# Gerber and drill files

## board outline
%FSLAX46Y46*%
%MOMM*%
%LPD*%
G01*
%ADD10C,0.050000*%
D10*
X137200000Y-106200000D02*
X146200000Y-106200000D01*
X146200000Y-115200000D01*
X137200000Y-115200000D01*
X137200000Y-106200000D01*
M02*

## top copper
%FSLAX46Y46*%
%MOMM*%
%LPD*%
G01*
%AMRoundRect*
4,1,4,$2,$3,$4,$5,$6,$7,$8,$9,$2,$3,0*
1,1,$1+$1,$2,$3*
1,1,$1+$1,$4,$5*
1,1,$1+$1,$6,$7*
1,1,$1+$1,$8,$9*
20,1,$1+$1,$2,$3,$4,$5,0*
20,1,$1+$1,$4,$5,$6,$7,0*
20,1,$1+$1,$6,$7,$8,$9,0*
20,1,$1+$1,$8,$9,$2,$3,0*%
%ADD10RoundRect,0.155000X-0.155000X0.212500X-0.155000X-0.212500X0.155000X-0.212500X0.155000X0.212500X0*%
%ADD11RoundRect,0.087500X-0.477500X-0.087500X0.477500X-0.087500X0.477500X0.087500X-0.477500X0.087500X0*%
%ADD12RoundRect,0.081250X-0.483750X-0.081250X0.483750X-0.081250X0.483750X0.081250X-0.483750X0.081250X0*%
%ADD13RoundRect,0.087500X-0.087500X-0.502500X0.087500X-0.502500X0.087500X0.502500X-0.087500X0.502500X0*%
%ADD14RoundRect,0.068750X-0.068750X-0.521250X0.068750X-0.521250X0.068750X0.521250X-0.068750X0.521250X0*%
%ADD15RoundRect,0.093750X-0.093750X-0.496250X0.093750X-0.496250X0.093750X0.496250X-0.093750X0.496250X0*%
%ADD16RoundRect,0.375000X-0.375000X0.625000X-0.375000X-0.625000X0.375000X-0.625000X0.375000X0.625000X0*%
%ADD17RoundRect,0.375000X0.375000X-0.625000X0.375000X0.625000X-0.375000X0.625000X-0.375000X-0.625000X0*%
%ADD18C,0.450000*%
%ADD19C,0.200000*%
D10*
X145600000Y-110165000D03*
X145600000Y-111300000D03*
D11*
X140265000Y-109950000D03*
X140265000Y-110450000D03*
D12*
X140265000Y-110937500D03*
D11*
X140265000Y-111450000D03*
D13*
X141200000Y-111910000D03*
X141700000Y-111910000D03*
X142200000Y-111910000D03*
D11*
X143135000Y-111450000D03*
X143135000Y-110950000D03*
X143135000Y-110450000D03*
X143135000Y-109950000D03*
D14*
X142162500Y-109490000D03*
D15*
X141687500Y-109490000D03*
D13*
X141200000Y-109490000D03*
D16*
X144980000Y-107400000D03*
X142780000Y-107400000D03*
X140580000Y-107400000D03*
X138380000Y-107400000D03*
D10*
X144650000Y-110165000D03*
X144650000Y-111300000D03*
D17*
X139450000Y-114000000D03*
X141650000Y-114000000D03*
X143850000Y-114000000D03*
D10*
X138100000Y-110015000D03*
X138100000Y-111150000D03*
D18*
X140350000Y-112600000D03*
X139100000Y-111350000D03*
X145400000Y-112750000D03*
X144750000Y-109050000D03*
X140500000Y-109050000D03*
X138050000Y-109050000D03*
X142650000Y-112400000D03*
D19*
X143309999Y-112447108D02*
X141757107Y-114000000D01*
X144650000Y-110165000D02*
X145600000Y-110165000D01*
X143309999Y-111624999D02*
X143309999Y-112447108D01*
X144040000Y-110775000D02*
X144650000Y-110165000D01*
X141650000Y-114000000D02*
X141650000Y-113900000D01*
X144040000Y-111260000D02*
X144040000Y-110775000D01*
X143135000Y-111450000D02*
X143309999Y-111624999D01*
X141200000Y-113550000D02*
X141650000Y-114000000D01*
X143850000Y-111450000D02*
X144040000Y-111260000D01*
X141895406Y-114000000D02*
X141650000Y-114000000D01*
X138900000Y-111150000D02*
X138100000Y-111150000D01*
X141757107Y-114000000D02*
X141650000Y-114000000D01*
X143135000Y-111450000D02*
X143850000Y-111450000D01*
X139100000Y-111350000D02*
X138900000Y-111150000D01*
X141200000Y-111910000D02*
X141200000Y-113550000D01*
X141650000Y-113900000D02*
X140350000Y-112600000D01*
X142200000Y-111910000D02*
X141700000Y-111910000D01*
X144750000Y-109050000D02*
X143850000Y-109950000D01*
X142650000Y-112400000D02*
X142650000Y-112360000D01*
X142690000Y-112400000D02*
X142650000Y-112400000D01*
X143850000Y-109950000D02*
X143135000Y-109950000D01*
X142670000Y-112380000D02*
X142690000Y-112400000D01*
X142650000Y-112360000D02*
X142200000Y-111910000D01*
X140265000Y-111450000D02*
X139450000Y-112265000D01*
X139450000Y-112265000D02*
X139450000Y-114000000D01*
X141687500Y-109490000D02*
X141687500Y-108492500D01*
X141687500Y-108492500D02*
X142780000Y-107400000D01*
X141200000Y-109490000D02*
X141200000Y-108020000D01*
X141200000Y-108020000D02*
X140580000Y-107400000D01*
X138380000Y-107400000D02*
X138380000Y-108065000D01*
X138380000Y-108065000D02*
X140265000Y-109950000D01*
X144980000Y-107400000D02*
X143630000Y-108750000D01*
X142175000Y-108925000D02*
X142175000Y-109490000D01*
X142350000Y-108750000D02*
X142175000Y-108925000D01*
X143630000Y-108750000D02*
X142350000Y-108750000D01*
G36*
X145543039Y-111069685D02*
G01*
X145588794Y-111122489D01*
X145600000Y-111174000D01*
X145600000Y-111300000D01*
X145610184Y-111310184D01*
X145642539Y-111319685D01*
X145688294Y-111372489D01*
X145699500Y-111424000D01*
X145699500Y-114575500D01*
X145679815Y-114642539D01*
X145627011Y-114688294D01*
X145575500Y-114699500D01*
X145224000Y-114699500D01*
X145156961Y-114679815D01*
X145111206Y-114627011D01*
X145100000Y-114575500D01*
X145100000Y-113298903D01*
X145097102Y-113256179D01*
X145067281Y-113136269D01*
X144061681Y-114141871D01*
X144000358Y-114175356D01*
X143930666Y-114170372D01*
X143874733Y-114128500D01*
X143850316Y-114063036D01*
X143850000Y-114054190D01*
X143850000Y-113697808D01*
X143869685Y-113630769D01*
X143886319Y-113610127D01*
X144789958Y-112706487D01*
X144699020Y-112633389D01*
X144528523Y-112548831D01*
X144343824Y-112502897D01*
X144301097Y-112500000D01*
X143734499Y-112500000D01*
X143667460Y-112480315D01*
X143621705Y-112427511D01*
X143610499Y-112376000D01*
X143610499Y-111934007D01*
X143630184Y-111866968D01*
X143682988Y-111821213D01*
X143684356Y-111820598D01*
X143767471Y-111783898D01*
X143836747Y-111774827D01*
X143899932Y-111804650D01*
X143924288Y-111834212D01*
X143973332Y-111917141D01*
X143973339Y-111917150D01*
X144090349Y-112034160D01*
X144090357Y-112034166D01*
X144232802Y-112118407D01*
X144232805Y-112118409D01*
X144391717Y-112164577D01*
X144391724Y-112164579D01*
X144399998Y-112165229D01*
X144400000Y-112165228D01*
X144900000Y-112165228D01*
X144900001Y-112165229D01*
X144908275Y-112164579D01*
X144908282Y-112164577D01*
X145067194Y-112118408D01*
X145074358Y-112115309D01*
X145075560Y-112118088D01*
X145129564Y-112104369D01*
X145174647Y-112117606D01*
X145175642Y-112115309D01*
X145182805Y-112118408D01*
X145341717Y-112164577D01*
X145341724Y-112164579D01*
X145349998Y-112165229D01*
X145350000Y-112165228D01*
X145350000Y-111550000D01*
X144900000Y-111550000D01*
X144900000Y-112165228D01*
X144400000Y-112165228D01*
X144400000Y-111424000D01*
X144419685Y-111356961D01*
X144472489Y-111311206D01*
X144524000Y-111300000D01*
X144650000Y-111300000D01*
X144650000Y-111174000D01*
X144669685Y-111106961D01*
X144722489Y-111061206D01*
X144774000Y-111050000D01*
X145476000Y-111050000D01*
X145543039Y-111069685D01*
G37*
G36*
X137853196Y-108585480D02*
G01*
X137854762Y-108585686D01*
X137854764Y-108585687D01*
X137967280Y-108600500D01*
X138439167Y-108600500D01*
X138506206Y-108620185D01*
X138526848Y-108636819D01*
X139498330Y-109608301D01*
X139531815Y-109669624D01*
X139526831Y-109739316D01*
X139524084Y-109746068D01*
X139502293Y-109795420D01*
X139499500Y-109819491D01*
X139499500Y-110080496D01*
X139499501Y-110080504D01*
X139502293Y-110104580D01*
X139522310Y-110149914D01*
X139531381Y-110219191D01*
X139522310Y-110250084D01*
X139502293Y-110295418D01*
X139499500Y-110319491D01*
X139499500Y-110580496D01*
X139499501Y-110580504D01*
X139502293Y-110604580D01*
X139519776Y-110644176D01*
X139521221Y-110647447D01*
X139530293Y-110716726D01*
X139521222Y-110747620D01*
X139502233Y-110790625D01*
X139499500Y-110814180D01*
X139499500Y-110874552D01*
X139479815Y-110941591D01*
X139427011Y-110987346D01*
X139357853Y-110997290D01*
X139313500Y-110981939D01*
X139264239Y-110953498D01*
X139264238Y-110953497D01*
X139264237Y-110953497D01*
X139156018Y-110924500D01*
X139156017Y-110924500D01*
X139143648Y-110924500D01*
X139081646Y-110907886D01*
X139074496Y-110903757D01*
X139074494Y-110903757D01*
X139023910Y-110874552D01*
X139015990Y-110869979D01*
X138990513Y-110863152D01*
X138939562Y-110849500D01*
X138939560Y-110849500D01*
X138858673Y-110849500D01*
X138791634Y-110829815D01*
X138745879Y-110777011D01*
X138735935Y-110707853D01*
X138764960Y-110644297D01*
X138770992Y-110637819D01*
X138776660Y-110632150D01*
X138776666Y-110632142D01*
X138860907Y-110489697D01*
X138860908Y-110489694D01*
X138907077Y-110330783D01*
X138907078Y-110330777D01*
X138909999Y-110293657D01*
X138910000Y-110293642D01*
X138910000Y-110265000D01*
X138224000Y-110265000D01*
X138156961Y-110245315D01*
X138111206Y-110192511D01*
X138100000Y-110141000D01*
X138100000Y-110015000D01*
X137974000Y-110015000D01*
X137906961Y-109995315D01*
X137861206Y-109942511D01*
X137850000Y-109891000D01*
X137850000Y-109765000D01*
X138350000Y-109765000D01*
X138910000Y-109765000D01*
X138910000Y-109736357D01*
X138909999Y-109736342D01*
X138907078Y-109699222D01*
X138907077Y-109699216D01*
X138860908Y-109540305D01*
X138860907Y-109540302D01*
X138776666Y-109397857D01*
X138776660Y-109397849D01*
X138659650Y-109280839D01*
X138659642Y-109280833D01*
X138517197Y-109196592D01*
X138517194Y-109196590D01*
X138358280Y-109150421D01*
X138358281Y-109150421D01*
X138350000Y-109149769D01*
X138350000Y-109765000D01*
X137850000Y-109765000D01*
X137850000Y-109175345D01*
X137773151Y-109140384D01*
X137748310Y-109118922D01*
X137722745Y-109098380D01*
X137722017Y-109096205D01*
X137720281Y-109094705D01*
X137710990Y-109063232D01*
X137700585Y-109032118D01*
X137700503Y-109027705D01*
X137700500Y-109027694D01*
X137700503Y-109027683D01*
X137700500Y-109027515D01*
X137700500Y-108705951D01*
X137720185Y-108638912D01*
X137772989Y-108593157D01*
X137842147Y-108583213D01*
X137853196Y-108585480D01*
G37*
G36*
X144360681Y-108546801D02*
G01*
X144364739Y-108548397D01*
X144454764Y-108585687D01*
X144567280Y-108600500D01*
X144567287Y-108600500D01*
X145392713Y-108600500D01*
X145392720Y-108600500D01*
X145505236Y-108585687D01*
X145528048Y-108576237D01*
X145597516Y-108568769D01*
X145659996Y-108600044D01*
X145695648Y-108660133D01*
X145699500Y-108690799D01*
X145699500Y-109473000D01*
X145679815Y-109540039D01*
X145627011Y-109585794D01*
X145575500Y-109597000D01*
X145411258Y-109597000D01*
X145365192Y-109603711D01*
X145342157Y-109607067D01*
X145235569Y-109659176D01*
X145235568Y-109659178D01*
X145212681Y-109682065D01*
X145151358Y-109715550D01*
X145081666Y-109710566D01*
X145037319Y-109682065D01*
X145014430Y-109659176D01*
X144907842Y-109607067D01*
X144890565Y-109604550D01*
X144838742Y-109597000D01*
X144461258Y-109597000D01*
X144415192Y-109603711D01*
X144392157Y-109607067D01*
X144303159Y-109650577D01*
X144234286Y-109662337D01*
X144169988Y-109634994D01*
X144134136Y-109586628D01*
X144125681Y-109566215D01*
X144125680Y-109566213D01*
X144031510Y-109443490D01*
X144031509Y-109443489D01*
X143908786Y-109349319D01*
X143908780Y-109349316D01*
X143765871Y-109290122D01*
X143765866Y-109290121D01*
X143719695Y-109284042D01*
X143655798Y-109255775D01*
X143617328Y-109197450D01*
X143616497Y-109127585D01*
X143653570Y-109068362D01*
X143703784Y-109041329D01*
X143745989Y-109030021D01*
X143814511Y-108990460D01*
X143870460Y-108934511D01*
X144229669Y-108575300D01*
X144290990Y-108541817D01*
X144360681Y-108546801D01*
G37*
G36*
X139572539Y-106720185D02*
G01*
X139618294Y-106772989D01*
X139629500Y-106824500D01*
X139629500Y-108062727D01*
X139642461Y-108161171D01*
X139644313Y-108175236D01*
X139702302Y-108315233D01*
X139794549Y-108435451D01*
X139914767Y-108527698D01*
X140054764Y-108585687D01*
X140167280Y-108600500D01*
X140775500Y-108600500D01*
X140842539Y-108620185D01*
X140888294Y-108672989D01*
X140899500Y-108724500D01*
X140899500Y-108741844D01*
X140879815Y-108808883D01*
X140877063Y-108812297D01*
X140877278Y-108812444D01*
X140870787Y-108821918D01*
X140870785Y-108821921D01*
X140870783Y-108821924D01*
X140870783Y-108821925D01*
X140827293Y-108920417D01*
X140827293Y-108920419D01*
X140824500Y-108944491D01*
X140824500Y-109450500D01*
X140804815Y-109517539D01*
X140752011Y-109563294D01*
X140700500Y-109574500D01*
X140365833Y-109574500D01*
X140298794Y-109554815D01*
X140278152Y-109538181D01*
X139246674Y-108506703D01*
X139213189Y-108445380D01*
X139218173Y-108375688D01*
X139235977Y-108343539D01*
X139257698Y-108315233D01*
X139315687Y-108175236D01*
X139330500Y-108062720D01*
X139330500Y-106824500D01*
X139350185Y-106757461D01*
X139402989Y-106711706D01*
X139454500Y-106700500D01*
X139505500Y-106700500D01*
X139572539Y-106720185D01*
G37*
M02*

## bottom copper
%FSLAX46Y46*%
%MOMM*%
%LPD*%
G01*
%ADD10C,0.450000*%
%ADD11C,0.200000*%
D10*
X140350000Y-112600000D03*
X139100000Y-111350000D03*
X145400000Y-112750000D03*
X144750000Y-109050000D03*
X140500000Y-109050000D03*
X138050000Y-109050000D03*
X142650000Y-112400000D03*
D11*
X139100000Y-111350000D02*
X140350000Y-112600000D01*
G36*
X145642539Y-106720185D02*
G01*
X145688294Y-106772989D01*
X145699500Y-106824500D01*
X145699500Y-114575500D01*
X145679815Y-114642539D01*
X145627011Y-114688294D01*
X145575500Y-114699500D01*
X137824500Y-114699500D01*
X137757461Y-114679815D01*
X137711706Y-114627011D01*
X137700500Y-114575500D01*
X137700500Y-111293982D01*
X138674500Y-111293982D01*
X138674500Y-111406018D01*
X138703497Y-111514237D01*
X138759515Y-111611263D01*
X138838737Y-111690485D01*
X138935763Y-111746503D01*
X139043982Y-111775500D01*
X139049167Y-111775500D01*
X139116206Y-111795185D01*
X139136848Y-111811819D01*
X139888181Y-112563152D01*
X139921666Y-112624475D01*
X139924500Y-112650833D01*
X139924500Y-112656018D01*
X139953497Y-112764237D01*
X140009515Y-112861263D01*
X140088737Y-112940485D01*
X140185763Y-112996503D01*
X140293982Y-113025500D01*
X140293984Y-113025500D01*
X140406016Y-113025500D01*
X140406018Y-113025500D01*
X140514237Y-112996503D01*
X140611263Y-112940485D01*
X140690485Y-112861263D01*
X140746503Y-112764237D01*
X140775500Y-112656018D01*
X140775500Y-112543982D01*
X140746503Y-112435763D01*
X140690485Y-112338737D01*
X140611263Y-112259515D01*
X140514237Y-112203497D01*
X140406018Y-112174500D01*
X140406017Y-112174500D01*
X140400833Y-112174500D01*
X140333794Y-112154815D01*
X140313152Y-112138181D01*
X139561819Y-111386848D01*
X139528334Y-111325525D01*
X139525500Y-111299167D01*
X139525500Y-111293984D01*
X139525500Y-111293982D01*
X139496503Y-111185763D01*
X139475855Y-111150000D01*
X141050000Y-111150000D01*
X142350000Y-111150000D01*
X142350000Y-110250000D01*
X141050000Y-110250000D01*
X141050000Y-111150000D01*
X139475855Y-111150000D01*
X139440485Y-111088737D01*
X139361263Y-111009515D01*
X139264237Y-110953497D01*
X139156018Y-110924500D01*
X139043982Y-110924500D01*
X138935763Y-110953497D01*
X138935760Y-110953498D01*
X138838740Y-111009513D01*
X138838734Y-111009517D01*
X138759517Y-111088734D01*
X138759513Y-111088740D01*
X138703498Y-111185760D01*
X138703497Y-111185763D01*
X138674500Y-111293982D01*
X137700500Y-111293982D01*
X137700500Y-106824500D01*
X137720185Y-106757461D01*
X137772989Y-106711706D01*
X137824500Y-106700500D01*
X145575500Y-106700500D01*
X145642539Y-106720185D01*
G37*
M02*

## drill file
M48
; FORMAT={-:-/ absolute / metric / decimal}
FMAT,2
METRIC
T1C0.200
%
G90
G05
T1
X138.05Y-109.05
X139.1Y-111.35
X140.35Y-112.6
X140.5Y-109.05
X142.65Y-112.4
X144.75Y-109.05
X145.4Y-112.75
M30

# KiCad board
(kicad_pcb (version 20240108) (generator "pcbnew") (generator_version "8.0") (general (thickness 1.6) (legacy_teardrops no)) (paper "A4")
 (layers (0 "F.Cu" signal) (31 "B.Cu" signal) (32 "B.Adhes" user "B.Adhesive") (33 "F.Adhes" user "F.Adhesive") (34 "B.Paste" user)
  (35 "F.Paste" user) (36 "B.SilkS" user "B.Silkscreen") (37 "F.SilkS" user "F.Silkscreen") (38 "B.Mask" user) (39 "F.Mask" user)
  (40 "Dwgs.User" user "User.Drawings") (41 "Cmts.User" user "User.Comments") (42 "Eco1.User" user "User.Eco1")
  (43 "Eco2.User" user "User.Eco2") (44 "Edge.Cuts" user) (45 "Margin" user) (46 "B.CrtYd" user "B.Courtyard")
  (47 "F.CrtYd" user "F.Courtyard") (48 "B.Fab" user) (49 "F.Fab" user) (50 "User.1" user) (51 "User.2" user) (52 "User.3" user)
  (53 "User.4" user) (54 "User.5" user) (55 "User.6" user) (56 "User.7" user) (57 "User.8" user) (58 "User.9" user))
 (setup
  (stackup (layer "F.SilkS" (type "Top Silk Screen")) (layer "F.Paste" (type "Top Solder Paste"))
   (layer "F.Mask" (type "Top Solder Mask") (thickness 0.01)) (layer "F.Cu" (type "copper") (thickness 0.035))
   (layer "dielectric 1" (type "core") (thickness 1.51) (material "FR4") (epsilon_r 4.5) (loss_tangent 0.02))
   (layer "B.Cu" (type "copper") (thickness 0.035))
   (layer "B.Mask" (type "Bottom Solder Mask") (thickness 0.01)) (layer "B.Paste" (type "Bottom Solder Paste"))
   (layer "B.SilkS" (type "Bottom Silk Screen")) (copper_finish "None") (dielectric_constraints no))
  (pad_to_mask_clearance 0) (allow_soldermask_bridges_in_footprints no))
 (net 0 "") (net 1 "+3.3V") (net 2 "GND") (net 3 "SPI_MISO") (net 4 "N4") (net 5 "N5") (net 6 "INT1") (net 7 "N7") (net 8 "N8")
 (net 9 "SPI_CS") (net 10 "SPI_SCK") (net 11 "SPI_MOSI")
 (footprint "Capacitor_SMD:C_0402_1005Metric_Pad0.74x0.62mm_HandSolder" (layer "F.Cu") (at 145.6 110.7325 -90)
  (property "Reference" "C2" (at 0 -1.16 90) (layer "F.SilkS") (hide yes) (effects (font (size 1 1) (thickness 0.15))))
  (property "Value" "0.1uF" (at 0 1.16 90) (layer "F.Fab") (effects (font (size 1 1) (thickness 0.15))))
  (pad "1" smd roundrect (at -0.5675 0 270) (size 0.735 0.62) (layers "F.Cu" "F.Paste" "F.Mask") (roundrect_rratio 0.25) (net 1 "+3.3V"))
  (pad "2" smd roundrect (at 0.5675 0 270) (size 0.735 0.62) (layers "F.Cu" "F.Paste" "F.Mask") (roundrect_rratio 0.25) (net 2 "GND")))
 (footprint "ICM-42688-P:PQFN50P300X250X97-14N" (layer "F.Cu") (at 141.7 110.7)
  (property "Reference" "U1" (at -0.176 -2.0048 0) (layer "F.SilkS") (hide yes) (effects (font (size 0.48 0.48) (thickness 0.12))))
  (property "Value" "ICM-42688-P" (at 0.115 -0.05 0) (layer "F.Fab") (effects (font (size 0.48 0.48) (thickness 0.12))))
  (pad "1" smd roundrect (at -1.435 -0.75) (size 1.13 0.35) (layers "F.Cu" "F.Paste") (roundrect_rratio 0.25) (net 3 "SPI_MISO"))
  (pad "2" smd roundrect (at -1.435 -0.25) (size 1.13 0.35) (layers "F.Cu" "F.Paste") (roundrect_rratio 0.25) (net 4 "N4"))
  (pad "3" smd roundrect (at -1.435 0.2375) (size 1.13 0.325) (layers "F.Cu" "F.Paste") (roundrect_rratio 0.25) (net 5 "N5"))
  (pad "4" smd roundrect (at -1.435 0.75) (size 1.13 0.35) (layers "F.Cu" "F.Paste") (roundrect_rratio 0.25) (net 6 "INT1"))
  (pad "5" smd roundrect (at -0.5 1.21) (size 0.35 1.18) (layers "F.Cu" "F.Paste") (roundrect_rratio 0.25) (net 1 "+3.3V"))
  (pad "6" smd roundrect (at 0 1.21) (size 0.35 1.18) (layers "F.Cu" "F.Paste") (roundrect_rratio 0.25) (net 2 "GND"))
  (pad "7" smd roundrect (at 0.5 1.21) (size 0.35 1.18) (layers "F.Cu" "F.Paste") (roundrect_rratio 0.25) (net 2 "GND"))
  (pad "8" smd roundrect (at 1.435 0.75) (size 1.13 0.35) (layers "F.Cu" "F.Paste") (roundrect_rratio 0.25) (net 1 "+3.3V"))
  (pad "9" smd roundrect (at 1.435 0.25) (size 1.13 0.35) (layers "F.Cu" "F.Paste") (roundrect_rratio 0.25) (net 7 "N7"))
  (pad "10" smd roundrect (at 1.435 -0.25) (size 1.13 0.35) (layers "F.Cu" "F.Paste") (roundrect_rratio 0.25) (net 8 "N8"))
  (pad "11" smd roundrect (at 1.435 -0.75) (size 1.13 0.35) (layers "F.Cu" "F.Paste") (roundrect_rratio 0.25) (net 2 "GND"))
  (pad "12" smd roundrect (at 0.4625 -1.21) (size 0.275 1.18) (layers "F.Cu" "F.Paste") (roundrect_rratio 0.25) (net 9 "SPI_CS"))
  (pad "13" smd roundrect (at -0.0125 -1.21) (size 0.375 1.18) (layers "F.Cu" "F.Paste") (roundrect_rratio 0.25) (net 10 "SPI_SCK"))
  (pad "14" smd roundrect (at -0.5 -1.21) (size 0.35 1.18) (layers "F.Cu" "F.Paste") (roundrect_rratio 0.25) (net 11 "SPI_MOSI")))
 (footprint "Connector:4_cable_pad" (layer "F.Cu") (at 145.78 106.2 180)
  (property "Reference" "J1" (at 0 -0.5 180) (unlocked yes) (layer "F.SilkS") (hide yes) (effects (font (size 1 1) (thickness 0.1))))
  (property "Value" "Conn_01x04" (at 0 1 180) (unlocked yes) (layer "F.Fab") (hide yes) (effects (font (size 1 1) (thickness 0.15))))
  (pad "1" smd roundrect (at 0.8 -1.2 270) (size 2 1.5) (layers "F.Cu" "F.Paste" "F.Mask") (roundrect_rratio 0.25) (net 9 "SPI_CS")
   (thermal_bridge_angle 45))
  (pad "2" smd roundrect (at 3 -1.2 270) (size 2 1.5) (layers "F.Cu" "F.Paste" "F.Mask") (roundrect_rratio 0.25) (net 10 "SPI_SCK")
   (thermal_bridge_angle 45))
  (pad "3" smd roundrect (at 5.2 -1.2 270) (size 2 1.5) (layers "F.Cu" "F.Paste" "F.Mask") (roundrect_rratio 0.25) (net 11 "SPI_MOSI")
   (thermal_bridge_angle 45))
  (pad "4" smd roundrect (at 7.4 -1.2 270) (size 2 1.5) (layers "F.Cu" "F.Paste" "F.Mask") (roundrect_rratio 0.25) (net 3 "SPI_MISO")
   (thermal_bridge_angle 45)))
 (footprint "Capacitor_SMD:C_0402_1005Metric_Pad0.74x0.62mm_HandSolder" (layer "F.Cu") (at 144.65 110.7325 -90)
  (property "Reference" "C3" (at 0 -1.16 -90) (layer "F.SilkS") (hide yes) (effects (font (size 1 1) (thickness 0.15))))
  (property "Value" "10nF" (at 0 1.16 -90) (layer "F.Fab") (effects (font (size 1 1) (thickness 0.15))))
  (pad "1" smd roundrect (at -0.5675 0 270) (size 0.735 0.62) (layers "F.Cu" "F.Paste" "F.Mask") (roundrect_rratio 0.25) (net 1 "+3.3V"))
  (pad "2" smd roundrect (at 0.5675 0 270) (size 0.735 0.62) (layers "F.Cu" "F.Paste" "F.Mask") (roundrect_rratio 0.25) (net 2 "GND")))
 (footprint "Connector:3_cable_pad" (layer "F.Cu") (at 138.65 115.2)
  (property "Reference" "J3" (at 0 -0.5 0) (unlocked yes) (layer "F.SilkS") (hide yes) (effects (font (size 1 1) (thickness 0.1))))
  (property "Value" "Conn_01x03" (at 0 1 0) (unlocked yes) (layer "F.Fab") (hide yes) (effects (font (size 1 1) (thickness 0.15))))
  (pad "1" smd roundrect (at 0.8 -1.2 90) (size 2 1.5) (layers "F.Cu" "F.Paste" "F.Mask") (roundrect_rratio 0.25) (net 6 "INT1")
   (thermal_bridge_angle 45))
  (pad "2" smd roundrect (at 3 -1.2 90) (size 2 1.5) (layers "F.Cu" "F.Paste" "F.Mask") (roundrect_rratio 0.25) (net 1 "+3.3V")
   (thermal_bridge_angle 45))
  (pad "3" smd roundrect (at 5.2 -1.2 90) (size 2 1.5) (layers "F.Cu" "F.Paste" "F.Mask") (roundrect_rratio 0.25) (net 2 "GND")
   (thermal_bridge_angle 45)))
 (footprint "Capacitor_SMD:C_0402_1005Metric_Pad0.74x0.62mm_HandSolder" (layer "F.Cu") (at 138.1 110.5825 -90)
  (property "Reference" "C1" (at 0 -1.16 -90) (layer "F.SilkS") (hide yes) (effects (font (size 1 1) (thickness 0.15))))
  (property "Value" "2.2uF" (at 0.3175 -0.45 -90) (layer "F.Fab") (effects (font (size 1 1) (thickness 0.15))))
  (pad "1" smd roundrect (at -0.5675 0 270) (size 0.735 0.62) (layers "F.Cu" "F.Paste" "F.Mask") (roundrect_rratio 0.25) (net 2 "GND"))
  (pad "2" smd roundrect (at 0.5675 0 270) (size 0.735 0.62) (layers "F.Cu" "F.Paste" "F.Mask") (roundrect_rratio 0.25) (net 1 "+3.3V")))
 (gr_rect (start 137.2 106.2) (end 146.2 115.2) (stroke (width 0.05) (type default)) (fill none) (layer "Edge.Cuts"))
 (segment (start 143.309999 112.447108) (end 141.757107 114) (width 0.2) (layer "F.Cu") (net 1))
 (segment (start 144.65 110.165) (end 145.6 110.165) (width 0.2) (layer "F.Cu") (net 1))
 (segment (start 143.309999 111.624999) (end 143.309999 112.447108) (width 0.2) (layer "F.Cu") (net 1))
 (segment (start 144.04 110.775) (end 144.65 110.165) (width 0.2) (layer "F.Cu") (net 1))
 (segment (start 141.65 114) (end 141.65 113.9) (width 0.2) (layer "F.Cu") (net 1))
 (segment (start 144.04 111.26) (end 144.04 110.775) (width 0.2) (layer "F.Cu") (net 1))
 (segment (start 143.135 111.45) (end 143.309999 111.624999) (width 0.2) (layer "F.Cu") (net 1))
 (segment (start 141.2 113.55) (end 141.65 114) (width 0.2) (layer "F.Cu") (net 1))
 (segment (start 143.85 111.45) (end 144.04 111.26) (width 0.2) (layer "F.Cu") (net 1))
 (segment (start 141.895406 114) (end 141.65 114) (width 0.2) (layer "F.Cu") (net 1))
 (segment (start 138.9 111.15) (end 138.1 111.15) (width 0.2) (layer "F.Cu") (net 1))
 (segment (start 141.757107 114) (end 141.65 114) (width 0.2) (layer "F.Cu") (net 1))
 (segment (start 143.135 111.45) (end 143.85 111.45) (width 0.2) (layer "F.Cu") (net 1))
 (segment (start 139.1 111.35) (end 138.9 111.15) (width 0.2) (layer "F.Cu") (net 1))
 (segment (start 141.2 111.91) (end 141.2 113.55) (width 0.2) (layer "F.Cu") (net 1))
 (segment (start 141.65 113.9) (end 140.35 112.6) (width 0.2) (layer "F.Cu") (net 1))
 (via (at 140.35 112.6) (size 0.45) (drill 0.2) (layers "F.Cu" "B.Cu") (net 1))
 (via (at 139.1 111.35) (size 0.45) (drill 0.2) (layers "F.Cu" "B.Cu") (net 1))
 (segment (start 139.1 111.35) (end 140.35 112.6) (width 0.2) (layer "B.Cu") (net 1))
 (segment (start 142.2 111.91) (end 141.7 111.91) (width 0.2) (layer "F.Cu") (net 2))
 (segment (start 144.75 109.05) (end 143.85 109.95) (width 0.2) (layer "F.Cu") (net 2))
 (segment (start 142.65 112.4) (end 142.65 112.36) (width 0.2) (layer "F.Cu") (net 2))
 (segment (start 142.69 112.4) (end 142.65 112.4) (width 0.2) (layer "F.Cu") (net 2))
 (segment (start 143.85 109.95) (end 143.135 109.95) (width 0.2) (layer "F.Cu") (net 2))
 (segment (start 142.67 112.38) (end 142.69 112.4) (width 0.2) (layer "F.Cu") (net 2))
 (segment (start 142.65 112.36) (end 142.2 111.91) (width 0.2) (layer "F.Cu") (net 2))
 (via (at 145.4 112.75) (size 0.45) (drill 0.2) (layers "F.Cu" "B.Cu") (free yes) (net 2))
 (via (at 144.75 109.05) (size 0.45) (drill 0.2) (layers "F.Cu" "B.Cu") (free yes) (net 2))
 (via (at 140.5 109.05) (size 0.45) (drill 0.2) (layers "F.Cu" "B.Cu") (free yes) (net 2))
 (via (at 138.05 109.05) (size 0.45) (drill 0.2) (layers "F.Cu" "B.Cu") (free yes) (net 2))
 (via (at 142.65 112.4) (size 0.45) (drill 0.2) (layers "F.Cu" "B.Cu") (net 2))
 (segment (start 140.265 111.45) (end 139.45 112.265) (width 0.2) (layer "F.Cu") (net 6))
 (segment (start 139.45 112.265) (end 139.45 114) (width 0.2) (layer "F.Cu") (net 6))
 (segment (start 141.6875 109.49) (end 141.6875 108.4925) (width 0.2) (layer "F.Cu") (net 10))
 (segment (start 141.6875 108.4925) (end 142.78 107.4) (width 0.2) (layer "F.Cu") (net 10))
 (segment (start 141.2 109.49) (end 141.2 108.02) (width 0.2) (layer "F.Cu") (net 11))
 (segment (start 141.2 108.02) (end 140.58 107.4) (width 0.2) (layer "F.Cu") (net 11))
 (segment (start 138.38 107.4) (end 138.38 108.065) (width 0.2) (layer "F.Cu") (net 3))
 (segment (start 138.38 108.065) (end 140.265 109.95) (width 0.2) (layer "F.Cu") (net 3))
 (segment (start 144.98 107.4) (end 143.63 108.75) (width 0.2) (layer "F.Cu") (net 9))
 (segment (start 142.175 108.925) (end 142.175 109.49) (width 0.2) (layer "F.Cu") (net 9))
 (segment (start 142.35 108.75) (end 142.175 108.925) (width 0.2) (layer "F.Cu") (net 9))
 (segment (start 143.63 108.75) (end 142.35 108.75) (width 0.2) (layer "F.Cu") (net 9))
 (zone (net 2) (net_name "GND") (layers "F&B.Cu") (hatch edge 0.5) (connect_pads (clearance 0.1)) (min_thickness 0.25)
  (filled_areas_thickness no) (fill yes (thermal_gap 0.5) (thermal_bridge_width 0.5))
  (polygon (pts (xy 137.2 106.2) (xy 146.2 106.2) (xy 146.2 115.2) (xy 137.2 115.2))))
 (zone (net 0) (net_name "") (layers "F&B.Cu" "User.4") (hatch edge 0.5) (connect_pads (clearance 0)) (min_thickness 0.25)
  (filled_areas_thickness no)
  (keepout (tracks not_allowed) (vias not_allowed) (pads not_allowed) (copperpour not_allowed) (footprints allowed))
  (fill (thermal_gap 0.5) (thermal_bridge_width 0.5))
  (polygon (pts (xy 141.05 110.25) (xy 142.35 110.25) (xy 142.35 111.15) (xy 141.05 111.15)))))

